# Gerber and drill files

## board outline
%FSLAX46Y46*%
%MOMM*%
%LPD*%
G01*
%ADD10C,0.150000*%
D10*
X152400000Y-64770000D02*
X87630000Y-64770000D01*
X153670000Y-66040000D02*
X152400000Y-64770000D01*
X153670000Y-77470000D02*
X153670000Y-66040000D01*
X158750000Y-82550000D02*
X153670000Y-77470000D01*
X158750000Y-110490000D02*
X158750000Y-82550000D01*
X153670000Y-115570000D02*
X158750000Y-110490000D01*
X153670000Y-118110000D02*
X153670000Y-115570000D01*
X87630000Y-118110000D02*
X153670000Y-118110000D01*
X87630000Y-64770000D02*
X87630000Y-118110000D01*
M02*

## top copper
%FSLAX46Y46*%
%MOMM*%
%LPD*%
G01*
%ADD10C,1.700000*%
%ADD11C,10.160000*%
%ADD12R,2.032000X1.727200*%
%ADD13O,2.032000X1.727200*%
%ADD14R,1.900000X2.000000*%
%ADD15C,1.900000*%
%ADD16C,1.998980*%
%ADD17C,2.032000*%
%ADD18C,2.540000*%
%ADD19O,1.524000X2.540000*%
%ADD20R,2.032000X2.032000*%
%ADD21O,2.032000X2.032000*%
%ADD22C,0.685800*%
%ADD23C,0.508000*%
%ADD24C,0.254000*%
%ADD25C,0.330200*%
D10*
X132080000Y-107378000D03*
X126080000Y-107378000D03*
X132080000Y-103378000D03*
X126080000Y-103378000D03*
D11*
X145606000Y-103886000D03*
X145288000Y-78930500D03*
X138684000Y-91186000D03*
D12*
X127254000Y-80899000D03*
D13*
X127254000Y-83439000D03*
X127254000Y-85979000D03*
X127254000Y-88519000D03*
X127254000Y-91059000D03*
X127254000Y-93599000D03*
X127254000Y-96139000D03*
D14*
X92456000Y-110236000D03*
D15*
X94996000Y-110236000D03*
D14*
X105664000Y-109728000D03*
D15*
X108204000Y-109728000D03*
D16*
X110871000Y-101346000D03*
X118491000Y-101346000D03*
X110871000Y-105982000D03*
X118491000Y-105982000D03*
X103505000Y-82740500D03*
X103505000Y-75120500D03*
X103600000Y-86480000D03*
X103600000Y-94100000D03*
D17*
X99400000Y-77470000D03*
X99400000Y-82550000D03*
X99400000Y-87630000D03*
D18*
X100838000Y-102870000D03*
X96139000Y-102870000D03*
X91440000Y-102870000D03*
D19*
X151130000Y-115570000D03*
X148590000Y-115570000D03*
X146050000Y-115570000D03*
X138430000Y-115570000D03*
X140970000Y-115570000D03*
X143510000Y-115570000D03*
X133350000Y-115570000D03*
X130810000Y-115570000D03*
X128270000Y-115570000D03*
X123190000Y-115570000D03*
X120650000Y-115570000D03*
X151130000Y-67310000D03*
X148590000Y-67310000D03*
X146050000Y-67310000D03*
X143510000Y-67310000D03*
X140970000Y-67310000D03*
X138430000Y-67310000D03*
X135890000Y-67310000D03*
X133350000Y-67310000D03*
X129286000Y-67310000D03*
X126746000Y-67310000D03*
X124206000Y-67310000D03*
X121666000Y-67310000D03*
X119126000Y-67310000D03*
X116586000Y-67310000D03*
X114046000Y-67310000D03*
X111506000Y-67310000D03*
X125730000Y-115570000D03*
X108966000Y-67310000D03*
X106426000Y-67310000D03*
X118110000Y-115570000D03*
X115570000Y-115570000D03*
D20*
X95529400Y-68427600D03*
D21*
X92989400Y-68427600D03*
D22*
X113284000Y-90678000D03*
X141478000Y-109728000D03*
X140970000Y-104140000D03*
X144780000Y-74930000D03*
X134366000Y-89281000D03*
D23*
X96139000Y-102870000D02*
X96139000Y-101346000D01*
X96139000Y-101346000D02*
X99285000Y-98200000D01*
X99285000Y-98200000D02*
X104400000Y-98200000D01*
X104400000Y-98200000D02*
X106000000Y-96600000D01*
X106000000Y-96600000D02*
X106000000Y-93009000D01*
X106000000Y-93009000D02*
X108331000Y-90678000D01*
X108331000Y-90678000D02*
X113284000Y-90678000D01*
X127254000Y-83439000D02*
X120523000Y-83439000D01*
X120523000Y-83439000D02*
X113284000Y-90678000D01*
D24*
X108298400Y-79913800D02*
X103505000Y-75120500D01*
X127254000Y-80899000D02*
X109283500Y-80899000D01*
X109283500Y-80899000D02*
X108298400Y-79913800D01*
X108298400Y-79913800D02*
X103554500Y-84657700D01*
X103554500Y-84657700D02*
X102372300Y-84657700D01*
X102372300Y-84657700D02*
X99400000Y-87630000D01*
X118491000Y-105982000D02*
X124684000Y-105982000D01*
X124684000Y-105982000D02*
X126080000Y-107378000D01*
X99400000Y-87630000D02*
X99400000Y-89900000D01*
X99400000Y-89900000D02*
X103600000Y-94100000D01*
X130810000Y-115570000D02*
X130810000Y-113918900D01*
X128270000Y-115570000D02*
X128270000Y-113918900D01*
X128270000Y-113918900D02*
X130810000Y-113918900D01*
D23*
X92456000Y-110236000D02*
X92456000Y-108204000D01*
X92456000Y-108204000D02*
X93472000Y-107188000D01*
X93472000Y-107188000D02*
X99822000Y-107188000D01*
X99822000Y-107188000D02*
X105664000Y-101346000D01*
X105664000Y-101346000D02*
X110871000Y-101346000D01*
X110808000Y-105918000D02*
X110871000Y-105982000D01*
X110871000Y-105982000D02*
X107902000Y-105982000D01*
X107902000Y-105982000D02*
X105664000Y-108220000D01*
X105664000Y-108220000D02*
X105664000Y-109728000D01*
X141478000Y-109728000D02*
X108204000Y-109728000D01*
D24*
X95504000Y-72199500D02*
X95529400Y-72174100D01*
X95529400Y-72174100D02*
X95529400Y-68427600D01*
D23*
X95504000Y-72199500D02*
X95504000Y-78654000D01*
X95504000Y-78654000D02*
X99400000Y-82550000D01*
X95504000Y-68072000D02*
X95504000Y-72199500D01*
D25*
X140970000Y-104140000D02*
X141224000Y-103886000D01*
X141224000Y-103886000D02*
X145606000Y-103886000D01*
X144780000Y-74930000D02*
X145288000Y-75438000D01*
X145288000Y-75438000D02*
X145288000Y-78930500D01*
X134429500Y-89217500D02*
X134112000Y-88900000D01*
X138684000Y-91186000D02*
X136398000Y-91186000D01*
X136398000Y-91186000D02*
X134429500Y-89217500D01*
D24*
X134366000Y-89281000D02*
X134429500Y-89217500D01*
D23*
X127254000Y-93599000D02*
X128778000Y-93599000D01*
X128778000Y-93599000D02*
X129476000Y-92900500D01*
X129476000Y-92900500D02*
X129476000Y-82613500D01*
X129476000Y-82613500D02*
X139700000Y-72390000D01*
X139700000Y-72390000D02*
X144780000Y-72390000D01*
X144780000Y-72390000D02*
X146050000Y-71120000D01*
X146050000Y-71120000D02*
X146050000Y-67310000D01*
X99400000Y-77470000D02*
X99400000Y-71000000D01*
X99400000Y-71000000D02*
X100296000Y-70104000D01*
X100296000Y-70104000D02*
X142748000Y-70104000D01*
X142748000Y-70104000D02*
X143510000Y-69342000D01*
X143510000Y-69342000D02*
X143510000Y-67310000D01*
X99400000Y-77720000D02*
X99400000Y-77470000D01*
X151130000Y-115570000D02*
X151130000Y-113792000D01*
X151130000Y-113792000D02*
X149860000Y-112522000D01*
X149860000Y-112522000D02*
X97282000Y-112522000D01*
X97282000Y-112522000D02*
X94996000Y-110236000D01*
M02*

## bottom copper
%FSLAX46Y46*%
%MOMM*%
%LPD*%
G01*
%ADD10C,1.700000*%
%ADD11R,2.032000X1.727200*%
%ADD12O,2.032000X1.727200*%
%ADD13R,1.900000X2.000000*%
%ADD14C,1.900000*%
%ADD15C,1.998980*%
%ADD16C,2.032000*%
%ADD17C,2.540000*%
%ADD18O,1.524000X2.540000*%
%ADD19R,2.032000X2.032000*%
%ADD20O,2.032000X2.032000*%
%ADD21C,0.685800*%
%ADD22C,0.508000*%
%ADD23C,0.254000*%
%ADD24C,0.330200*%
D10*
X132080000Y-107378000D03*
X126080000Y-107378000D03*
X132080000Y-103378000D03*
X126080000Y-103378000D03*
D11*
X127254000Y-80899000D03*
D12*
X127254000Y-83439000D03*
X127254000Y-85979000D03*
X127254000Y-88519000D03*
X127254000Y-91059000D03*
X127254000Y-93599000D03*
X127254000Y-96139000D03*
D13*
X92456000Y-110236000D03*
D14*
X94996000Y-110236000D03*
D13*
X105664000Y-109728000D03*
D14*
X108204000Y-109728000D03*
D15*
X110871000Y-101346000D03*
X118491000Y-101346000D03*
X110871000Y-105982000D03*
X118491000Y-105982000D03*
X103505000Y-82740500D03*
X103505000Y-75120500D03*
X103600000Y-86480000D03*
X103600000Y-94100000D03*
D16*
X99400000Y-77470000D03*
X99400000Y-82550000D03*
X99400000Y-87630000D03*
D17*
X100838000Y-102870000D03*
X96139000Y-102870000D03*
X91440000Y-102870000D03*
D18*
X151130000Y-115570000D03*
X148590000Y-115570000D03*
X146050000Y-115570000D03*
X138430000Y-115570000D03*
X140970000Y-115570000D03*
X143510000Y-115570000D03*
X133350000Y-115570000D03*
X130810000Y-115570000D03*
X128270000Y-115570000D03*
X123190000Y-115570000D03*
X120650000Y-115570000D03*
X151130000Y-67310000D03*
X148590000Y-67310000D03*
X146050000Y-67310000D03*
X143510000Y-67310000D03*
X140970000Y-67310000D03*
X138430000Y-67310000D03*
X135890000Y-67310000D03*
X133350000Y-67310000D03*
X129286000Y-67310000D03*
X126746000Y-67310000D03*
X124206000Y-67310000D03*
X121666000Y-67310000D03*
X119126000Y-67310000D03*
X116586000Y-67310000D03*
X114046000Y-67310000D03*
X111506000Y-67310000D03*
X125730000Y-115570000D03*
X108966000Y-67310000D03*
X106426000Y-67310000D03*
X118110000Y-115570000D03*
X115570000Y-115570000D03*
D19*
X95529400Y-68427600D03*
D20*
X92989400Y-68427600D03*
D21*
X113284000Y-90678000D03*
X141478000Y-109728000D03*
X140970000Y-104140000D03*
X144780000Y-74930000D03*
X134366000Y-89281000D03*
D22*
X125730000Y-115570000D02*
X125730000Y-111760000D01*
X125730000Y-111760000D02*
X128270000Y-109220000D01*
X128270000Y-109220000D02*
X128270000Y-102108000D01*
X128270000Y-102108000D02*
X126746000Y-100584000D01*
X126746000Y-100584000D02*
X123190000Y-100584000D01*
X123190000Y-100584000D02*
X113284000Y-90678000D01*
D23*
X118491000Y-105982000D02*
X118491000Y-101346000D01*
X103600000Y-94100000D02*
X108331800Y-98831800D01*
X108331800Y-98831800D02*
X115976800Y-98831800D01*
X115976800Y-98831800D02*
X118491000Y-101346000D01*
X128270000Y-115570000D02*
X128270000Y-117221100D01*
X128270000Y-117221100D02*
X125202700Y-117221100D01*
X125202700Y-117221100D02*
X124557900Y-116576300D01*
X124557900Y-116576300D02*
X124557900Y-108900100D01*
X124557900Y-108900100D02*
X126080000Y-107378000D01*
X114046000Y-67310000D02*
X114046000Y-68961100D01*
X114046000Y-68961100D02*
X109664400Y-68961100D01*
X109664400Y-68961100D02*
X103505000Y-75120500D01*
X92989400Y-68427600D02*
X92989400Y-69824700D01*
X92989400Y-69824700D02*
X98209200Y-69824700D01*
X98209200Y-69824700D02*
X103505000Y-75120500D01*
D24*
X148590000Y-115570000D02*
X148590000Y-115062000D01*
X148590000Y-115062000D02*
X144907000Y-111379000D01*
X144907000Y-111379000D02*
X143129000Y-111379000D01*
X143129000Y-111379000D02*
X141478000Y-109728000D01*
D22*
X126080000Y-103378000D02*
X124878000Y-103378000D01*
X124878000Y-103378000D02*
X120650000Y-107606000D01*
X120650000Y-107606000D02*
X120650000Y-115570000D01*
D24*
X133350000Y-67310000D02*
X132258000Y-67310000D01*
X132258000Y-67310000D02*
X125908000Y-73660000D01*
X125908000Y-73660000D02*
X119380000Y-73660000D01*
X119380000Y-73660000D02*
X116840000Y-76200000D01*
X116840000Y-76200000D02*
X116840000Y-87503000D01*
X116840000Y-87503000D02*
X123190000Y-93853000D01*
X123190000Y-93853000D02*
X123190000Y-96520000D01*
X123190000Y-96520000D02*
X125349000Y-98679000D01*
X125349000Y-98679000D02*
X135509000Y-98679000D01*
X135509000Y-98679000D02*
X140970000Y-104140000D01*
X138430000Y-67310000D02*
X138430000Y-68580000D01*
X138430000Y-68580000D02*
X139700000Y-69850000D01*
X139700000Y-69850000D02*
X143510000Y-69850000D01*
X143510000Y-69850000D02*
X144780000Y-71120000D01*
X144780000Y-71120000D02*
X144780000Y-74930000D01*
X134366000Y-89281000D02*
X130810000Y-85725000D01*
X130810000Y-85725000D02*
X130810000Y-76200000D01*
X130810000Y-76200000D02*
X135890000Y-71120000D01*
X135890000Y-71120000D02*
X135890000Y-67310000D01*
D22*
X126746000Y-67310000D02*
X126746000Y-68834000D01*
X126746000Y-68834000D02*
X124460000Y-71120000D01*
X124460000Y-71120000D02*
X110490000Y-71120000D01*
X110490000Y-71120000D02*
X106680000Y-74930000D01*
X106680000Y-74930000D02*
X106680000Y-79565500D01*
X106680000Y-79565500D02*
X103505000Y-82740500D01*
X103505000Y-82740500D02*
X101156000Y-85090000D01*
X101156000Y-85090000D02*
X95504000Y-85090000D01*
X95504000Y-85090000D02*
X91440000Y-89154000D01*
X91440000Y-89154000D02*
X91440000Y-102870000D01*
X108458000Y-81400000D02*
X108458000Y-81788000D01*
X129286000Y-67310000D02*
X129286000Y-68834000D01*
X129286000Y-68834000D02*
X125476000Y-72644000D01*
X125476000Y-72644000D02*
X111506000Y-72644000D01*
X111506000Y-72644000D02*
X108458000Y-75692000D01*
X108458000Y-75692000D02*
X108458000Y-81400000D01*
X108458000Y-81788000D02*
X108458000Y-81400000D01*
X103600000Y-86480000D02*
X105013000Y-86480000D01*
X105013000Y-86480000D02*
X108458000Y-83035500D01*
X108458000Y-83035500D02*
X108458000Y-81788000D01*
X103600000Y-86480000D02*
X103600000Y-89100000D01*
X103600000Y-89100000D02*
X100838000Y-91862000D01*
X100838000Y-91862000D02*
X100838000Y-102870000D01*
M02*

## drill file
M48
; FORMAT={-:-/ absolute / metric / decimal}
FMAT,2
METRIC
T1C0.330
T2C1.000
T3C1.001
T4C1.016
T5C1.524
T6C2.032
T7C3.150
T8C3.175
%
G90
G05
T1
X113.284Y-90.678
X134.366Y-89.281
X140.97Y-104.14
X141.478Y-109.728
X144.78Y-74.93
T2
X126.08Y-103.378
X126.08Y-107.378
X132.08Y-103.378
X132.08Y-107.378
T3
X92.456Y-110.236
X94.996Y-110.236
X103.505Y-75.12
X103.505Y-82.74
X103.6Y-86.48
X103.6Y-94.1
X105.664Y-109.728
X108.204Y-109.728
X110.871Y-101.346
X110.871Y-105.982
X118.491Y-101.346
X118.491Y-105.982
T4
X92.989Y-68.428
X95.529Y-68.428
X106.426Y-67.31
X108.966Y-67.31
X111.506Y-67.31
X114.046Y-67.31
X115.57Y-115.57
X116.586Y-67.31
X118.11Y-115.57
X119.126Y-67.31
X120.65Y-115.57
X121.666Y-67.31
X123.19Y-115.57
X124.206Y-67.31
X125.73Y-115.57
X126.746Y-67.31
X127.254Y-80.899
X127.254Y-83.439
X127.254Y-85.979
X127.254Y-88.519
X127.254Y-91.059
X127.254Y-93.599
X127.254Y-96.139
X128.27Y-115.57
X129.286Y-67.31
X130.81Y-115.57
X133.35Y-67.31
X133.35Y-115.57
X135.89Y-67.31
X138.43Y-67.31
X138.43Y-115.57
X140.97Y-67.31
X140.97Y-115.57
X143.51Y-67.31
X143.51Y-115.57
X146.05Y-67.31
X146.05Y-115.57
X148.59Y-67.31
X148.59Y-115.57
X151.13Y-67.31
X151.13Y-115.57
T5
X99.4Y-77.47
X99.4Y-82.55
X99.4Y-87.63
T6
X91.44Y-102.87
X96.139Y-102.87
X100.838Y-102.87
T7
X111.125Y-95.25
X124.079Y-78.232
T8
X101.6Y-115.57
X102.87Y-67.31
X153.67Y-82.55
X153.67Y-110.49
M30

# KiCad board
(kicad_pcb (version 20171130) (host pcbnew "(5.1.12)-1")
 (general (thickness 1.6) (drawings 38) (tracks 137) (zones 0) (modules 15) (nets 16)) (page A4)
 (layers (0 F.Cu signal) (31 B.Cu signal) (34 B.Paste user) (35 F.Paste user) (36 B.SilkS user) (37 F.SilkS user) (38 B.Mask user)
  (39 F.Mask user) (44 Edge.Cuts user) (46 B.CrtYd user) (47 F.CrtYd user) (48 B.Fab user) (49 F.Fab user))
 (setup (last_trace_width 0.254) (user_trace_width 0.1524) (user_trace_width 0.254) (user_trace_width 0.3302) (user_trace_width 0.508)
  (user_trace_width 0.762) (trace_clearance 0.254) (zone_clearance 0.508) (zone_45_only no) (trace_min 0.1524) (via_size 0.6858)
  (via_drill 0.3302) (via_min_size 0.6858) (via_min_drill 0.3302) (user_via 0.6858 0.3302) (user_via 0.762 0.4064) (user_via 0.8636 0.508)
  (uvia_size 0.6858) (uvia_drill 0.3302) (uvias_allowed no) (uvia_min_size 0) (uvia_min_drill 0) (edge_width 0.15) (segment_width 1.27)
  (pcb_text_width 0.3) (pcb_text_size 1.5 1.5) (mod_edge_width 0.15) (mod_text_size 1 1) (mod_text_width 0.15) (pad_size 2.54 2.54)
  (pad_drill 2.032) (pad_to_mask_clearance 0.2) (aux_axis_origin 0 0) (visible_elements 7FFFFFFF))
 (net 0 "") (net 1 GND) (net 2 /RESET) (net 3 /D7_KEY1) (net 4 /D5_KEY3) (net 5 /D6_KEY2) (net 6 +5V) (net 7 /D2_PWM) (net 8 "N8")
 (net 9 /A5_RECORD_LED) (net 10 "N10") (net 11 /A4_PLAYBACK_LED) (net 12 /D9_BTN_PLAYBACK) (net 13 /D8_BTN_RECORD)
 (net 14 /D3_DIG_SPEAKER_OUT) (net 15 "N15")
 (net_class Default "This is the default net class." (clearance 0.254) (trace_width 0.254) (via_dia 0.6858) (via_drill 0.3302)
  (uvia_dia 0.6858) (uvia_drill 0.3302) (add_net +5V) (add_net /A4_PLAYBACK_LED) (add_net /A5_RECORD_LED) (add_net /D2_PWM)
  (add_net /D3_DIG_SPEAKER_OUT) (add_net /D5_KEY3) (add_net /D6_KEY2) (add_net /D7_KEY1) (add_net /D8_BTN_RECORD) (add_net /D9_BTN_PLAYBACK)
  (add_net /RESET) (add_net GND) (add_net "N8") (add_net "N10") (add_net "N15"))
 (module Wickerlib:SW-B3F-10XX (layer F.Cu) (at 126.08 103.378)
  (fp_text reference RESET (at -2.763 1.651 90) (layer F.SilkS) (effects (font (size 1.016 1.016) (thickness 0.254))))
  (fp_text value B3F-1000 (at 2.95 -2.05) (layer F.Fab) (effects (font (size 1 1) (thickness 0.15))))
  (pad 4 thru_hole circle (at 6 4) (size 1.7 1.7) (drill 1) (layers *.Cu *.Mask))
  (pad 3 thru_hole circle (at 0 4) (size 1.7 1.7) (drill 1) (layers *.Cu *.Mask) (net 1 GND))
  (pad 2 thru_hole circle (at 6 0) (size 1.7 1.7) (drill 1) (layers *.Cu *.Mask))
  (pad 1 thru_hole circle (at 0 0) (size 1.7 1.7) (drill 1) (layers *.Cu *.Mask) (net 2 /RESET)))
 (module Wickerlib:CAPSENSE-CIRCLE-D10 (layer F.Cu) (at 145.606 103.886)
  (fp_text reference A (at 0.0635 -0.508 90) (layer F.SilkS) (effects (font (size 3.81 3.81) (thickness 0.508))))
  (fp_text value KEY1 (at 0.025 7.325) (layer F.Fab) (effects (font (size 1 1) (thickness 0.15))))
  (pad 1 smd circle (at 0 0) (size 10.16 10.16) (layers F.Cu) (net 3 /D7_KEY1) (clearance 0.508)))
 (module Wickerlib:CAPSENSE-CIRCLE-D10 (layer F.Cu) (at 145.288 78.9305)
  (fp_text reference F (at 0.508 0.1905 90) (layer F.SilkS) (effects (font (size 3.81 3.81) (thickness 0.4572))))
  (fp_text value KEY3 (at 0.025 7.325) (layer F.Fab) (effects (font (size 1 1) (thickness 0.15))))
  (pad 1 smd circle (at 0 0) (size 10.16 10.16) (layers F.Cu) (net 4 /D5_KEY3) (clearance 0.508)))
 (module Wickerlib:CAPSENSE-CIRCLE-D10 (layer F.Cu) (at 138.684 91.186)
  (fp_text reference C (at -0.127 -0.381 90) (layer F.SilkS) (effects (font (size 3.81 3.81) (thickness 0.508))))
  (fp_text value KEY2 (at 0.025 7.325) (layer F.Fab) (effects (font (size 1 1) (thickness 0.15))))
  (pad 1 smd circle (at 0 0) (size 10.16 10.16) (layers F.Cu) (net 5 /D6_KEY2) (clearance 0.508)))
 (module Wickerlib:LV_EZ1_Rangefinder (layer F.Cu) (at 108.585 97.79)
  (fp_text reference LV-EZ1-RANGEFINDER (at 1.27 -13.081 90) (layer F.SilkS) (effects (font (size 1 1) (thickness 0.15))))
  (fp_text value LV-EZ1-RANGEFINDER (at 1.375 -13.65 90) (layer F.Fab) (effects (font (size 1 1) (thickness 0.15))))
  (pad "" np_thru_hole circle (at 15.494 -19.558) (size 3.1496 3.1496) (drill 3.1496) (layers F.Cu))
  (pad 1 thru_hole rect (at 18.669 -16.891) (size 2.032 1.7272) (drill 1.016) (layers *.Cu *.Mask F.SilkS) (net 1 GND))
  (pad 2 thru_hole oval (at 18.669 -14.351) (size 2.032 1.7272) (drill 1.016) (layers *.Cu *.Mask F.SilkS) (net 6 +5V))
  (pad 3 thru_hole oval (at 18.669 -11.811) (size 2.032 1.7272) (drill 1.016) (layers *.Cu *.Mask F.SilkS))
  (pad 4 thru_hole oval (at 18.669 -9.271) (size 2.032 1.7272) (drill 1.016) (layers *.Cu *.Mask F.SilkS))
  (pad 5 thru_hole oval (at 18.669 -6.731) (size 2.032 1.7272) (drill 1.016) (layers *.Cu *.Mask F.SilkS))
  (pad 6 thru_hole oval (at 18.669 -4.191) (size 2.032 1.7272) (drill 1.016) (layers *.Cu *.Mask F.SilkS) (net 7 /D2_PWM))
  (pad 7 thru_hole oval (at 18.669 -1.651) (size 2.032 1.7272) (drill 1.016) (layers *.Cu *.Mask F.SilkS))
  (pad "" np_thru_hole circle (at 2.54 -2.54) (size 3.1496 3.1496) (drill 3.1496) (layers F.Cu)))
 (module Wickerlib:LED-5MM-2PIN (layer F.Cu) (at 92.456 110.236)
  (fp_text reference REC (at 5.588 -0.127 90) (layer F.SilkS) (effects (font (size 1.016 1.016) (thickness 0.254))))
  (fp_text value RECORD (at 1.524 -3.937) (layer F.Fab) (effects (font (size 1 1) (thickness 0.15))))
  (pad 1 thru_hole rect (at 0 0 90) (size 2 1.9) (drill 1.00076) (layers *.Cu *.Mask F.SilkS) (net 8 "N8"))
  (pad 2 thru_hole circle (at 2.54 0) (size 1.9 1.9) (drill 1.00076) (layers *.Cu *.Mask F.SilkS) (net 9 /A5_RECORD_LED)))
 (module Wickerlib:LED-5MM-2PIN (layer F.Cu) (at 105.664 109.728)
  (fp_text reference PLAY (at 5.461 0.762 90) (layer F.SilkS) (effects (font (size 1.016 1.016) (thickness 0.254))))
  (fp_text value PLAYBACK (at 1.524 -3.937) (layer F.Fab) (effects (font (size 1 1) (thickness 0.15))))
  (pad 1 thru_hole rect (at 0 0 90) (size 2 1.9) (drill 1.00076) (layers *.Cu *.Mask F.SilkS) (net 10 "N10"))
  (pad 2 thru_hole circle (at 2.54 0) (size 1.9 1.9) (drill 1.00076) (layers *.Cu *.Mask F.SilkS) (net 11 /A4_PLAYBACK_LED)))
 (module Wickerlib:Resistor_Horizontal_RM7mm (layer F.Cu) (at 110.871 101.346)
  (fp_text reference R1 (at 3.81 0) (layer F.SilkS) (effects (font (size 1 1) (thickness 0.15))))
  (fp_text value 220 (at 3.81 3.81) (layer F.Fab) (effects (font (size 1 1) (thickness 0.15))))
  (pad 1 thru_hole circle (at 0 0) (size 1.99898 1.99898) (drill 1.00076) (layers *.Cu *.SilkS *.Mask) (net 8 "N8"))
  (pad 2 thru_hole circle (at 7.62 0) (size 1.99898 1.99898) (drill 1.00076) (layers *.Cu *.SilkS *.Mask) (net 1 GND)))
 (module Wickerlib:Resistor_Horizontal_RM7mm (layer F.Cu) (at 110.871 105.982)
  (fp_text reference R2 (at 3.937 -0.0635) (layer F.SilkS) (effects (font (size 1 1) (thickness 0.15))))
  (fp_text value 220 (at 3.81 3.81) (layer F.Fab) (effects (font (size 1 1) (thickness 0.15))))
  (pad 1 thru_hole circle (at 0 0) (size 1.99898 1.99898) (drill 1.00076) (layers *.Cu *.SilkS *.Mask) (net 10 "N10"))
  (pad 2 thru_hole circle (at 7.62 0) (size 1.99898 1.99898) (drill 1.00076) (layers *.Cu *.SilkS *.Mask) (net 1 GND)))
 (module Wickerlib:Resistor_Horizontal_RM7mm (layer F.Cu) (at 103.505 82.7405 90)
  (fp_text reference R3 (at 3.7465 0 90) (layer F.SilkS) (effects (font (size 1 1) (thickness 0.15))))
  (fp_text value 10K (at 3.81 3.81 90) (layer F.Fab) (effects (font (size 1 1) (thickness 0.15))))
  (pad 1 thru_hole circle (at 0 0 90) (size 1.99898 1.99898) (drill 1.00076) (layers *.Cu *.SilkS *.Mask) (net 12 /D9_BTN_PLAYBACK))
  (pad 2 thru_hole circle (at 7.62 0 90) (size 1.99898 1.99898) (drill 1.00076) (layers *.Cu *.SilkS *.Mask) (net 1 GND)))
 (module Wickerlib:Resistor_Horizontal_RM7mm (layer F.Cu) (at 103.6 86.48 270)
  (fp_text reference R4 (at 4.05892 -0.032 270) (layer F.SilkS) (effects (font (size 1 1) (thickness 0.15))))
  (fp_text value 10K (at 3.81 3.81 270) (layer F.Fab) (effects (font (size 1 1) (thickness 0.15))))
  (pad 1 thru_hole circle (at 0 0 270) (size 1.99898 1.99898) (drill 1.00076) (layers *.Cu *.SilkS *.Mask) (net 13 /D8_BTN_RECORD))
  (pad 2 thru_hole circle (at 7.62 0 270) (size 1.99898 1.99898) (drill 1.00076) (layers *.Cu *.SilkS *.Mask) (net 1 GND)))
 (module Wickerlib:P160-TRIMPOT (layer F.Cu) (at 99.4 77.47)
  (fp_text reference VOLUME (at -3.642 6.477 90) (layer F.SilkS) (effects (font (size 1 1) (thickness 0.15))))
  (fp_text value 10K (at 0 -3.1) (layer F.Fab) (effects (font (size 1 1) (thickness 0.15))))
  (pad 1 thru_hole circle (at 0 0) (size 2.032 2.032) (drill 1.524) (layers *.Cu *.Mask F.SilkS) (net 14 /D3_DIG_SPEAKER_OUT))
  (pad 2 thru_hole circle (at 0 5.08) (size 2.032 2.032) (drill 1.524) (layers *.Cu *.Mask F.SilkS) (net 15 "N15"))
  (pad 3 thru_hole circle (at 0 10.16) (size 2.032 2.032) (drill 1.524) (layers *.Cu *.Mask F.SilkS) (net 1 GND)))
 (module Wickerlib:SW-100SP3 (layer F.Cu) (at 100.838 102.87 270)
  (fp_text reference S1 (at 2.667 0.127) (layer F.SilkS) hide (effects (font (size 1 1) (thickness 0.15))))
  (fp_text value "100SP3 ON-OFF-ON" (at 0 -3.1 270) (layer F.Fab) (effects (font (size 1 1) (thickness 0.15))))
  (pad 1 thru_hole circle (at 0 0 270) (size 2.54 2.54) (drill 2.032) (layers *.Cu *.Mask F.SilkS) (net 13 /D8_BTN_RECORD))
  (pad 2 thru_hole circle (at 0 4.699 270) (size 2.54 2.54) (drill 2.032) (layers *.Cu *.Mask F.SilkS) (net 6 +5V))
  (pad 3 thru_hole circle (at 0 9.398 270) (size 2.54 2.54) (drill 2.032) (layers *.Cu *.Mask F.SilkS) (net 12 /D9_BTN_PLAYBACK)))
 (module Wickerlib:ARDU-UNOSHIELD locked (layer F.Cu) (at 87.63 118.11)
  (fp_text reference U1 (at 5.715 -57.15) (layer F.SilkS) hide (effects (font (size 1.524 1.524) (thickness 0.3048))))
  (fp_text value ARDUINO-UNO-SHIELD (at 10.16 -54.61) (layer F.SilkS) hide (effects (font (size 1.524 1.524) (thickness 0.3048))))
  (pad A5 thru_hole oval (at 63.5 -2.54 90) (size 2.54 1.524) (drill 1.016) (layers *.Cu *.Mask F.SilkS) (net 9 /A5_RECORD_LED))
  (pad A4 thru_hole oval (at 60.96 -2.54 90) (size 2.54 1.524) (drill 1.016) (layers *.Cu *.Mask F.SilkS) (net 11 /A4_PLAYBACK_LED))
  (pad A3 thru_hole oval (at 58.42 -2.54 90) (size 2.54 1.524) (drill 1.016) (layers *.Cu *.Mask F.SilkS))
  (pad A0 thru_hole oval (at 50.8 -2.54 90) (size 2.54 1.524) (drill 1.016) (layers *.Cu *.Mask F.SilkS))
  (pad A1 thru_hole oval (at 53.34 -2.54 90) (size 2.54 1.524) (drill 1.016) (layers *.Cu *.Mask F.SilkS))
  (pad A2 thru_hole oval (at 55.88 -2.54 90) (size 2.54 1.524) (drill 1.016) (layers *.Cu *.Mask F.SilkS))
  (pad VIN thru_hole oval (at 45.72 -2.54 90) (size 2.54 1.524) (drill 1.016) (layers *.Cu *.Mask F.SilkS))
  (pad GND2 thru_hole oval (at 43.18 -2.54 90) (size 2.54 1.524) (drill 1.016) (layers *.Cu *.Mask F.SilkS) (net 1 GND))
  (pad GND1 thru_hole oval (at 40.64 -2.54 90) (size 2.54 1.524) (drill 1.016) (layers *.Cu *.Mask F.SilkS) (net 1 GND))
  (pad 3V3 thru_hole oval (at 35.56 -2.54 90) (size 2.54 1.524) (drill 1.016) (layers *.Cu *.Mask F.SilkS))
  (pad RST thru_hole oval (at 33.02 -2.54 90) (size 2.54 1.524) (drill 1.016) (layers *.Cu *.Mask F.SilkS) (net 2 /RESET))
  (pad D0 thru_hole oval (at 63.5 -50.8 90) (size 2.54 1.524) (drill 1.016) (layers *.Cu *.Mask F.SilkS))
  (pad D1 thru_hole oval (at 60.96 -50.8 90) (size 2.54 1.524) (drill 1.016) (layers *.Cu *.Mask F.SilkS))
  (pad D2 thru_hole oval (at 58.42 -50.8 90) (size 2.54 1.524) (drill 1.016) (layers *.Cu *.Mask F.SilkS) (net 7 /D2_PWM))
  (pad D3 thru_hole oval (at 55.88 -50.8 90) (size 2.54 1.524) (drill 1.016) (layers *.Cu *.Mask F.SilkS) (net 14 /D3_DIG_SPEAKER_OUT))
  (pad D4 thru_hole oval (at 53.34 -50.8 90) (size 2.54 1.524) (drill 1.016) (layers *.Cu *.Mask F.SilkS))
  (pad D5 thru_hole oval (at 50.8 -50.8 90) (size 2.54 1.524) (drill 1.016) (layers *.Cu *.Mask F.SilkS) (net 4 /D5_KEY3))
  (pad D6 thru_hole oval (at 48.26 -50.8 90) (size 2.54 1.524) (drill 1.016) (layers *.Cu *.Mask F.SilkS) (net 5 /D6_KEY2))
  (pad D7 thru_hole oval (at 45.72 -50.8 90) (size 2.54 1.524) (drill 1.016) (layers *.Cu *.Mask F.SilkS) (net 3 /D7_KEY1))
  (pad D8 thru_hole oval (at 41.656 -50.8 90) (size 2.54 1.524) (drill 1.016) (layers *.Cu *.Mask F.SilkS) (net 13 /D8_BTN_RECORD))
  (pad D9 thru_hole oval (at 39.116 -50.8 90) (size 2.54 1.524) (drill 1.016) (layers *.Cu *.Mask F.SilkS) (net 12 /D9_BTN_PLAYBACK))
  (pad D10 thru_hole oval (at 36.576 -50.8 90) (size 2.54 1.524) (drill 1.016) (layers *.Cu *.Mask F.SilkS))
  (pad D11 thru_hole oval (at 34.036 -50.8 90) (size 2.54 1.524) (drill 1.016) (layers *.Cu *.Mask F.SilkS))
  (pad D12 thru_hole oval (at 31.496 -50.8 90) (size 2.54 1.524) (drill 1.016) (layers *.Cu *.Mask F.SilkS))
  (pad D13 thru_hole oval (at 28.956 -50.8 90) (size 2.54 1.524) (drill 1.016) (layers *.Cu *.Mask F.SilkS))
  (pad GND3 thru_hole oval (at 26.416 -50.8 90) (size 2.54 1.524) (drill 1.016) (layers *.Cu *.Mask F.SilkS) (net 1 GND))
  (pad AREF thru_hole oval (at 23.876 -50.8 90) (size 2.54 1.524) (drill 1.016) (layers *.Cu *.Mask F.SilkS))
  (pad 5V thru_hole oval (at 38.1 -2.54 90) (size 2.54 1.524) (drill 1.016) (layers *.Cu *.Mask F.SilkS) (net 6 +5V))
  (pad "" np_thru_hole circle (at 66.04 -7.62 90) (size 3.175 3.175) (drill 3.175) (layers *.Cu *.Mask F.SilkS))
  (pad "" np_thru_hole circle (at 66.04 -35.56 90) (size 3.175 3.175) (drill 3.175) (layers *.Cu *.Mask F.SilkS))
  (pad "" np_thru_hole circle (at 15.24 -50.8 90) (size 3.175 3.175) (drill 3.175) (layers *.Cu *.Mask F.SilkS))
  (pad "" np_thru_hole circle (at 13.97 -2.54 90) (size 3.175 3.175) (drill 3.175) (layers *.Cu *.Mask F.SilkS))
  (pad SDA thru_hole oval (at 21.336 -50.8 90) (size 2.54 1.524) (drill 1.016) (layers *.Cu *.Mask F.SilkS))
  (pad SCL thru_hole oval (at 18.796 -50.8 90) (size 2.54 1.524) (drill 1.016) (layers *.Cu *.Mask F.SilkS))
  (pad IO thru_hole oval (at 30.48 -2.54 90) (size 2.54 1.524) (drill 1.016) (layers *.Cu *.Mask F.SilkS))
  (pad NC thru_hole oval (at 27.94 -2.54 90) (size 2.54 1.524) (drill 1.016) (layers *.Cu *.Mask F.SilkS)))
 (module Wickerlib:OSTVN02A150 (layer F.Cu) (at 95.5294 68.4276 270)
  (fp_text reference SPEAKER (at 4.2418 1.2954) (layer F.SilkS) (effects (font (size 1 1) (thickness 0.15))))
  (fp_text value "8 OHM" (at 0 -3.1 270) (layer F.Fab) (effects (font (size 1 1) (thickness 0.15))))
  (pad 1 thru_hole rect (at 0 0 270) (size 2.032 2.032) (drill 1.016) (layers *.Cu *.Mask F.SilkS) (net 15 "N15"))
  (pad 2 thru_hole oval (at 0 2.54 270) (size 2.032 2.032) (drill 1.016) (layers *.Cu *.Mask F.SilkS) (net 1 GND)))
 (gr_line (start 152.4 64.77) (end 87.63 64.77) (angle 90) (layer Edge.Cuts) (width 0.15))
 (gr_line (start 153.67 66.04) (end 152.4 64.77) (angle 90) (layer Edge.Cuts) (width 0.15))
 (gr_line (start 153.67 77.47) (end 153.67 66.04) (angle 90) (layer Edge.Cuts) (width 0.15))
 (gr_line (start 158.75 82.55) (end 153.67 77.47) (angle 90) (layer Edge.Cuts) (width 0.15))
 (gr_line (start 158.75 110.49) (end 158.75 82.55) (angle 90) (layer Edge.Cuts) (width 0.15))
 (gr_line (start 153.67 115.57) (end 158.75 110.49) (angle 90) (layer Edge.Cuts) (width 0.15))
 (gr_line (start 153.67 118.11) (end 153.67 115.57) (angle 90) (layer Edge.Cuts) (width 0.15))
 (gr_line (start 87.63 118.11) (end 153.67 118.11) (angle 90) (layer Edge.Cuts) (width 0.15))
 (gr_line (start 87.63 64.77) (end 87.63 118.11) (angle 90) (layer Edge.Cuts) (width 0.15))
 (segment (start 96.139 102.87) (end 96.139 101.346) (width 0.508) (layer F.Cu) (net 6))
 (segment (start 96.139 101.346) (end 99.285 98.2) (width 0.508) (layer F.Cu) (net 6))
 (segment (start 99.285 98.2) (end 104.4 98.2) (width 0.508) (layer F.Cu) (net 6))
 (segment (start 104.4 98.2) (end 106 96.6) (width 0.508) (layer F.Cu) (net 6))
 (segment (start 106 96.6) (end 106 93.009) (width 0.508) (layer F.Cu) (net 6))
 (segment (start 106 93.009) (end 108.331 90.678) (width 0.508) (layer F.Cu) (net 6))
 (segment (start 108.331 90.678) (end 113.284 90.678) (width 0.508) (layer F.Cu) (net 6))
 (segment (start 127.254 83.439) (end 120.523 83.439) (width 0.508) (layer F.Cu) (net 6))
 (segment (start 120.523 83.439) (end 113.284 90.678) (width 0.508) (layer F.Cu) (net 6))
 (segment (start 125.73 115.57) (end 125.73 111.76) (width 0.508) (layer B.Cu) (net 6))
 (segment (start 125.73 111.76) (end 128.27 109.22) (width 0.508) (layer B.Cu) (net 6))
 (segment (start 128.27 109.22) (end 128.27 102.108) (width 0.508) (layer B.Cu) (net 6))
 (segment (start 128.27 102.108) (end 126.746 100.584) (width 0.508) (layer B.Cu) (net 6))
 (segment (start 126.746 100.584) (end 123.19 100.584) (width 0.508) (layer B.Cu) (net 6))
 (segment (start 123.19 100.584) (end 113.284 90.678) (width 0.508) (layer B.Cu) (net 6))
 (via (at 113.284 90.678) (size 0.6858) (layers F.Cu B.Cu) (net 6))
 (segment (start 108.2984 79.9138) (end 103.505 75.1205) (width 0.254) (layer F.Cu) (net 1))
 (segment (start 127.254 80.899) (end 109.2835 80.899) (width 0.254) (layer F.Cu) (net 1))
 (segment (start 109.2835 80.899) (end 108.2984 79.9138) (width 0.254) (layer F.Cu) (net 1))
 (segment (start 108.2984 79.9138) (end 103.5545 84.6577) (width 0.254) (layer F.Cu) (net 1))
 (segment (start 103.5545 84.6577) (end 102.3723 84.6577) (width 0.254) (layer F.Cu) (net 1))
 (segment (start 102.3723 84.6577) (end 99.4 87.63) (width 0.254) (layer F.Cu) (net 1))
 (segment (start 118.491 105.982) (end 124.684 105.982) (width 0.254) (layer F.Cu) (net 1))
 (segment (start 124.684 105.982) (end 126.08 107.378) (width 0.254) (layer F.Cu) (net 1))
 (segment (start 118.491 105.982) (end 118.491 101.346) (width 0.254) (layer B.Cu) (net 1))
 (segment (start 103.6 94.1) (end 108.3318 98.8318) (width 0.254) (layer B.Cu) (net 1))
 (segment (start 108.3318 98.8318) (end 115.9768 98.8318) (width 0.254) (layer B.Cu) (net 1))
 (segment (start 115.9768 98.8318) (end 118.491 101.346) (width 0.254) (layer B.Cu) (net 1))
 (segment (start 99.4 87.63) (end 99.4 89.9) (width 0.254) (layer F.Cu) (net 1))
 (segment (start 99.4 89.9) (end 103.6 94.1) (width 0.254) (layer F.Cu) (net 1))
 (segment (start 128.27 115.57) (end 128.27 117.2211) (width 0.254) (layer B.Cu) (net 1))
 (segment (start 128.27 117.2211) (end 125.2027 117.2211) (width 0.254) (layer B.Cu) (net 1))
 (segment (start 125.2027 117.2211) (end 124.5579 116.5763) (width 0.254) (layer B.Cu) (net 1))
 (segment (start 124.5579 116.5763) (end 124.5579 108.9001) (width 0.254) (layer B.Cu) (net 1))
 (segment (start 124.5579 108.9001) (end 126.08 107.378) (width 0.254) (layer B.Cu) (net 1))
 (segment (start 130.81 115.57) (end 130.81 113.9189) (width 0.254) (layer F.Cu) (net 1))
 (segment (start 128.27 115.57) (end 128.27 113.9189) (width 0.254) (layer F.Cu) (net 1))
 (segment (start 128.27 113.9189) (end 130.81 113.9189) (width 0.254) (layer F.Cu) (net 1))
 (segment (start 114.046 67.31) (end 114.046 68.9611) (width 0.254) (layer B.Cu) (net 1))
 (segment (start 114.046 68.9611) (end 109.6644 68.9611) (width 0.254) (layer B.Cu) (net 1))
 (segment (start 109.6644 68.9611) (end 103.505 75.1205) (width 0.254) (layer B.Cu) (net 1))
 (segment (start 92.9894 68.4276) (end 92.9894 69.8247) (width 0.254) (layer B.Cu) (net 1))
 (segment (start 92.9894 69.8247) (end 98.2092 69.8247) (width 0.254) (layer B.Cu) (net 1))
 (segment (start 98.2092 69.8247) (end 103.505 75.1205) (width 0.254) (layer B.Cu) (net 1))
 (segment (start 92.456 110.236) (end 92.456 108.204) (width 0.508) (layer F.Cu) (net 8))
 (segment (start 92.456 108.204) (end 93.472 107.188) (width 0.508) (layer F.Cu) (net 8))
 (segment (start 93.472 107.188) (end 99.822 107.188) (width 0.508) (layer F.Cu) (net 8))
 (segment (start 99.822 107.188) (end 105.664 101.346) (width 0.508) (layer F.Cu) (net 8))
 (segment (start 105.664 101.346) (end 110.871 101.346) (width 0.508) (layer F.Cu) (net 8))
 (segment (start 110.808 105.918) (end 110.871 105.982) (width 0.508) (layer F.Cu) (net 10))
 (segment (start 110.871 105.982) (end 107.902 105.982) (width 0.508) (layer F.Cu) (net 10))
 (segment (start 107.902 105.982) (end 105.664 108.22) (width 0.508) (layer F.Cu) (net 10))
 (segment (start 105.664 108.22) (end 105.664 109.728) (width 0.508) (layer F.Cu) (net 10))
 (segment (start 148.59 115.57) (end 148.59 115.062) (width 0.3302) (layer B.Cu) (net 11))
 (segment (start 148.59 115.062) (end 144.907 111.379) (width 0.3302) (layer B.Cu) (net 11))
 (segment (start 144.907 111.379) (end 143.129 111.379) (width 0.3302) (layer B.Cu) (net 11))
 (segment (start 143.129 111.379) (end 141.478 109.728) (width 0.3302) (layer B.Cu) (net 11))
 (segment (start 141.478 109.728) (end 108.204 109.728) (width 0.508) (layer F.Cu) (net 11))
 (via (at 141.478 109.728) (size 0.6858) (layers F.Cu B.Cu) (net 11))
 (segment (start 126.08 103.378) (end 124.878 103.378) (width 0.508) (layer B.Cu) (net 2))
 (segment (start 124.878 103.378) (end 120.65 107.606) (width 0.508) (layer B.Cu) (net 2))
 (segment (start 120.65 107.606) (end 120.65 115.57) (width 0.508) (layer B.Cu) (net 2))
 (segment (start 95.504 72.1995) (end 95.5294 72.1741) (width 0.254) (layer F.Cu) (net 15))
 (segment (start 95.5294 72.1741) (end 95.5294 68.4276) (width 0.254) (layer F.Cu) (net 15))
 (segment (start 95.504 72.1995) (end 95.504 78.654) (width 0.508) (layer F.Cu) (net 15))
 (segment (start 95.504 78.654) (end 99.4 82.55) (width 0.508) (layer F.Cu) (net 15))
 (segment (start 95.504 68.072) (end 95.504 72.1995) (width 0.508) (layer F.Cu) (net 15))
 (segment (start 140.97 104.14) (end 141.224 103.886) (width 0.3302) (layer F.Cu) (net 3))
 (segment (start 141.224 103.886) (end 145.606 103.886) (width 0.3302) (layer F.Cu) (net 3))
 (segment (start 133.35 67.31) (end 132.258 67.31) (width 0.3302) (layer B.Cu) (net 3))
 (segment (start 132.258 67.31) (end 125.908 73.66) (width 0.3302) (layer B.Cu) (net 3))
 (segment (start 125.908 73.66) (end 119.38 73.66) (width 0.3302) (layer B.Cu) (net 3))
 (segment (start 119.38 73.66) (end 116.84 76.2) (width 0.3302) (layer B.Cu) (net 3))
 (segment (start 116.84 76.2) (end 116.84 87.503) (width 0.3302) (layer B.Cu) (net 3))
 (segment (start 116.84 87.503) (end 123.19 93.853) (width 0.3302) (layer B.Cu) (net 3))
 (segment (start 123.19 93.853) (end 123.19 96.52) (width 0.3302) (layer B.Cu) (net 3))
 (segment (start 123.19 96.52) (end 125.349 98.679) (width 0.3302) (layer B.Cu) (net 3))
 (segment (start 125.349 98.679) (end 135.509 98.679) (width 0.3302) (layer B.Cu) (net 3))
 (segment (start 135.509 98.679) (end 140.97 104.14) (width 0.3302) (layer B.Cu) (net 3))
 (via (at 140.97 104.14) (size 0.6858) (layers F.Cu B.Cu) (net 3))
 (segment (start 144.78 74.93) (end 145.288 75.438) (width 0.3302) (layer F.Cu) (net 4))
 (segment (start 145.288 75.438) (end 145.288 78.9305) (width 0.3302) (layer F.Cu) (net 4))
 (segment (start 138.43 67.31) (end 138.43 68.58) (width 0.3302) (layer B.Cu) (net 4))
 (segment (start 138.43 68.58) (end 139.7 69.85) (width 0.3302) (layer B.Cu) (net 4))
 (segment (start 139.7 69.85) (end 143.51 69.85) (width 0.3302) (layer B.Cu) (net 4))
 (segment (start 143.51 69.85) (end 144.78 71.12) (width 0.3302) (layer B.Cu) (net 4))
 (segment (start 144.78 71.12) (end 144.78 74.93) (width 0.3302) (layer B.Cu) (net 4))
 (via (at 144.78 74.93) (size 0.6858) (layers F.Cu B.Cu) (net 4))
 (segment (start 134.4295 89.2175) (end 134.112 88.9) (width 0.3302) (layer F.Cu) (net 5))
 (segment (start 138.684 91.186) (end 136.398 91.186) (width 0.3302) (layer F.Cu) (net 5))
 (segment (start 136.398 91.186) (end 134.4295 89.2175) (width 0.3302) (layer F.Cu) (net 5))
 (segment (start 134.366 89.281) (end 134.4295 89.2175) (width 0.254) (layer F.Cu) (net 5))
 (segment (start 134.366 89.281) (end 130.81 85.725) (width 0.3302) (layer B.Cu) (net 5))
 (segment (start 130.81 85.725) (end 130.81 76.2) (width 0.3302) (layer B.Cu) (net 5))
 (segment (start 130.81 76.2) (end 135.89 71.12) (width 0.3302) (layer B.Cu) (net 5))
 (segment (start 135.89 71.12) (end 135.89 67.31) (width 0.3302) (layer B.Cu) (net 5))
 (via (at 134.366 89.281) (size 0.6858) (layers F.Cu B.Cu) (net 5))
 (segment (start 127.254 93.599) (end 128.778 93.599) (width 0.508) (layer F.Cu) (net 7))
 (segment (start 128.778 93.599) (end 129.476 92.9005) (width 0.508) (layer F.Cu) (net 7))
 (segment (start 129.476 92.9005) (end 129.476 82.6135) (width 0.508) (layer F.Cu) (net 7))
 (segment (start 129.476 82.6135) (end 139.7 72.39) (width 0.508) (layer F.Cu) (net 7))
 (segment (start 139.7 72.39) (end 144.78 72.39) (width 0.508) (layer F.Cu) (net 7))
 (segment (start 144.78 72.39) (end 146.05 71.12) (width 0.508) (layer F.Cu) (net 7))
 (segment (start 146.05 71.12) (end 146.05 67.31) (width 0.508) (layer F.Cu) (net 7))
 (segment (start 99.4 77.47) (end 99.4 71) (width 0.508) (layer F.Cu) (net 14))
 (segment (start 99.4 71) (end 100.296 70.104) (width 0.508) (layer F.Cu) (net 14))
 (segment (start 100.296 70.104) (end 142.748 70.104) (width 0.508) (layer F.Cu) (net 14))
 (segment (start 142.748 70.104) (end 143.51 69.342) (width 0.508) (layer F.Cu) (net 14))
 (segment (start 143.51 69.342) (end 143.51 67.31) (width 0.508) (layer F.Cu) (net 14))
 (segment (start 99.4 77.72) (end 99.4 77.47) (width 0.508) (layer F.Cu) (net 14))
 (segment (start 151.13 115.57) (end 151.13 113.792) (width 0.508) (layer F.Cu) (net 9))
 (segment (start 151.13 113.792) (end 149.86 112.522) (width 0.508) (layer F.Cu) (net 9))
 (segment (start 149.86 112.522) (end 97.282 112.522) (width 0.508) (layer F.Cu) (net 9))
 (segment (start 97.282 112.522) (end 94.996 110.236) (width 0.508) (layer F.Cu) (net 9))
 (segment (start 126.746 67.31) (end 126.746 68.834) (width 0.508) (layer B.Cu) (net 12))
 (segment (start 126.746 68.834) (end 124.46 71.12) (width 0.508) (layer B.Cu) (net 12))
 (segment (start 124.46 71.12) (end 110.49 71.12) (width 0.508) (layer B.Cu) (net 12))
 (segment (start 110.49 71.12) (end 106.68 74.93) (width 0.508) (layer B.Cu) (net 12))
 (segment (start 106.68 74.93) (end 106.68 79.5655) (width 0.508) (layer B.Cu) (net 12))
 (segment (start 106.68 79.5655) (end 103.505 82.7405) (width 0.508) (layer B.Cu) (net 12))
 (segment (start 103.505 82.7405) (end 101.156 85.09) (width 0.508) (layer B.Cu) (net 12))
 (segment (start 101.156 85.09) (end 95.504 85.09) (width 0.508) (layer B.Cu) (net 12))
 (segment (start 95.504 85.09) (end 91.44 89.154) (width 0.508) (layer B.Cu) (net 12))
 (segment (start 91.44 89.154) (end 91.44 102.87) (width 0.508) (layer B.Cu) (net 12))
 (segment (start 108.458 81.4) (end 108.458 81.788) (width 0.508) (layer B.Cu) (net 13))
 (segment (start 129.286 67.31) (end 129.286 68.834) (width 0.508) (layer B.Cu) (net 13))
 (segment (start 129.286 68.834) (end 125.476 72.644) (width 0.508) (layer B.Cu) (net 13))
 (segment (start 125.476 72.644) (end 111.506 72.644) (width 0.508) (layer B.Cu) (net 13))
 (segment (start 111.506 72.644) (end 108.458 75.692) (width 0.508) (layer B.Cu) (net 13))
 (segment (start 108.458 75.692) (end 108.458 81.4) (width 0.508) (layer B.Cu) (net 13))
 (segment (start 108.458 81.788) (end 108.458 81.4) (width 0.508) (layer B.Cu) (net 13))
 (segment (start 103.6 86.48) (end 105.013 86.48) (width 0.508) (layer B.Cu) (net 13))
 (segment (start 105.013 86.48) (end 108.458 83.0355) (width 0.508) (layer B.Cu) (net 13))
 (segment (start 108.458 83.0355) (end 108.458 81.788) (width 0.508) (layer B.Cu) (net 13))
 (segment (start 103.6 86.48) (end 103.6 89.1) (width 0.508) (layer B.Cu) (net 13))
 (segment (start 103.6 89.1) (end 100.838 91.862) (width 0.508) (layer B.Cu) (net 13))
 (segment (start 100.838 91.862) (end 100.838 102.87) (width 0.508) (layer B.Cu) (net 13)))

